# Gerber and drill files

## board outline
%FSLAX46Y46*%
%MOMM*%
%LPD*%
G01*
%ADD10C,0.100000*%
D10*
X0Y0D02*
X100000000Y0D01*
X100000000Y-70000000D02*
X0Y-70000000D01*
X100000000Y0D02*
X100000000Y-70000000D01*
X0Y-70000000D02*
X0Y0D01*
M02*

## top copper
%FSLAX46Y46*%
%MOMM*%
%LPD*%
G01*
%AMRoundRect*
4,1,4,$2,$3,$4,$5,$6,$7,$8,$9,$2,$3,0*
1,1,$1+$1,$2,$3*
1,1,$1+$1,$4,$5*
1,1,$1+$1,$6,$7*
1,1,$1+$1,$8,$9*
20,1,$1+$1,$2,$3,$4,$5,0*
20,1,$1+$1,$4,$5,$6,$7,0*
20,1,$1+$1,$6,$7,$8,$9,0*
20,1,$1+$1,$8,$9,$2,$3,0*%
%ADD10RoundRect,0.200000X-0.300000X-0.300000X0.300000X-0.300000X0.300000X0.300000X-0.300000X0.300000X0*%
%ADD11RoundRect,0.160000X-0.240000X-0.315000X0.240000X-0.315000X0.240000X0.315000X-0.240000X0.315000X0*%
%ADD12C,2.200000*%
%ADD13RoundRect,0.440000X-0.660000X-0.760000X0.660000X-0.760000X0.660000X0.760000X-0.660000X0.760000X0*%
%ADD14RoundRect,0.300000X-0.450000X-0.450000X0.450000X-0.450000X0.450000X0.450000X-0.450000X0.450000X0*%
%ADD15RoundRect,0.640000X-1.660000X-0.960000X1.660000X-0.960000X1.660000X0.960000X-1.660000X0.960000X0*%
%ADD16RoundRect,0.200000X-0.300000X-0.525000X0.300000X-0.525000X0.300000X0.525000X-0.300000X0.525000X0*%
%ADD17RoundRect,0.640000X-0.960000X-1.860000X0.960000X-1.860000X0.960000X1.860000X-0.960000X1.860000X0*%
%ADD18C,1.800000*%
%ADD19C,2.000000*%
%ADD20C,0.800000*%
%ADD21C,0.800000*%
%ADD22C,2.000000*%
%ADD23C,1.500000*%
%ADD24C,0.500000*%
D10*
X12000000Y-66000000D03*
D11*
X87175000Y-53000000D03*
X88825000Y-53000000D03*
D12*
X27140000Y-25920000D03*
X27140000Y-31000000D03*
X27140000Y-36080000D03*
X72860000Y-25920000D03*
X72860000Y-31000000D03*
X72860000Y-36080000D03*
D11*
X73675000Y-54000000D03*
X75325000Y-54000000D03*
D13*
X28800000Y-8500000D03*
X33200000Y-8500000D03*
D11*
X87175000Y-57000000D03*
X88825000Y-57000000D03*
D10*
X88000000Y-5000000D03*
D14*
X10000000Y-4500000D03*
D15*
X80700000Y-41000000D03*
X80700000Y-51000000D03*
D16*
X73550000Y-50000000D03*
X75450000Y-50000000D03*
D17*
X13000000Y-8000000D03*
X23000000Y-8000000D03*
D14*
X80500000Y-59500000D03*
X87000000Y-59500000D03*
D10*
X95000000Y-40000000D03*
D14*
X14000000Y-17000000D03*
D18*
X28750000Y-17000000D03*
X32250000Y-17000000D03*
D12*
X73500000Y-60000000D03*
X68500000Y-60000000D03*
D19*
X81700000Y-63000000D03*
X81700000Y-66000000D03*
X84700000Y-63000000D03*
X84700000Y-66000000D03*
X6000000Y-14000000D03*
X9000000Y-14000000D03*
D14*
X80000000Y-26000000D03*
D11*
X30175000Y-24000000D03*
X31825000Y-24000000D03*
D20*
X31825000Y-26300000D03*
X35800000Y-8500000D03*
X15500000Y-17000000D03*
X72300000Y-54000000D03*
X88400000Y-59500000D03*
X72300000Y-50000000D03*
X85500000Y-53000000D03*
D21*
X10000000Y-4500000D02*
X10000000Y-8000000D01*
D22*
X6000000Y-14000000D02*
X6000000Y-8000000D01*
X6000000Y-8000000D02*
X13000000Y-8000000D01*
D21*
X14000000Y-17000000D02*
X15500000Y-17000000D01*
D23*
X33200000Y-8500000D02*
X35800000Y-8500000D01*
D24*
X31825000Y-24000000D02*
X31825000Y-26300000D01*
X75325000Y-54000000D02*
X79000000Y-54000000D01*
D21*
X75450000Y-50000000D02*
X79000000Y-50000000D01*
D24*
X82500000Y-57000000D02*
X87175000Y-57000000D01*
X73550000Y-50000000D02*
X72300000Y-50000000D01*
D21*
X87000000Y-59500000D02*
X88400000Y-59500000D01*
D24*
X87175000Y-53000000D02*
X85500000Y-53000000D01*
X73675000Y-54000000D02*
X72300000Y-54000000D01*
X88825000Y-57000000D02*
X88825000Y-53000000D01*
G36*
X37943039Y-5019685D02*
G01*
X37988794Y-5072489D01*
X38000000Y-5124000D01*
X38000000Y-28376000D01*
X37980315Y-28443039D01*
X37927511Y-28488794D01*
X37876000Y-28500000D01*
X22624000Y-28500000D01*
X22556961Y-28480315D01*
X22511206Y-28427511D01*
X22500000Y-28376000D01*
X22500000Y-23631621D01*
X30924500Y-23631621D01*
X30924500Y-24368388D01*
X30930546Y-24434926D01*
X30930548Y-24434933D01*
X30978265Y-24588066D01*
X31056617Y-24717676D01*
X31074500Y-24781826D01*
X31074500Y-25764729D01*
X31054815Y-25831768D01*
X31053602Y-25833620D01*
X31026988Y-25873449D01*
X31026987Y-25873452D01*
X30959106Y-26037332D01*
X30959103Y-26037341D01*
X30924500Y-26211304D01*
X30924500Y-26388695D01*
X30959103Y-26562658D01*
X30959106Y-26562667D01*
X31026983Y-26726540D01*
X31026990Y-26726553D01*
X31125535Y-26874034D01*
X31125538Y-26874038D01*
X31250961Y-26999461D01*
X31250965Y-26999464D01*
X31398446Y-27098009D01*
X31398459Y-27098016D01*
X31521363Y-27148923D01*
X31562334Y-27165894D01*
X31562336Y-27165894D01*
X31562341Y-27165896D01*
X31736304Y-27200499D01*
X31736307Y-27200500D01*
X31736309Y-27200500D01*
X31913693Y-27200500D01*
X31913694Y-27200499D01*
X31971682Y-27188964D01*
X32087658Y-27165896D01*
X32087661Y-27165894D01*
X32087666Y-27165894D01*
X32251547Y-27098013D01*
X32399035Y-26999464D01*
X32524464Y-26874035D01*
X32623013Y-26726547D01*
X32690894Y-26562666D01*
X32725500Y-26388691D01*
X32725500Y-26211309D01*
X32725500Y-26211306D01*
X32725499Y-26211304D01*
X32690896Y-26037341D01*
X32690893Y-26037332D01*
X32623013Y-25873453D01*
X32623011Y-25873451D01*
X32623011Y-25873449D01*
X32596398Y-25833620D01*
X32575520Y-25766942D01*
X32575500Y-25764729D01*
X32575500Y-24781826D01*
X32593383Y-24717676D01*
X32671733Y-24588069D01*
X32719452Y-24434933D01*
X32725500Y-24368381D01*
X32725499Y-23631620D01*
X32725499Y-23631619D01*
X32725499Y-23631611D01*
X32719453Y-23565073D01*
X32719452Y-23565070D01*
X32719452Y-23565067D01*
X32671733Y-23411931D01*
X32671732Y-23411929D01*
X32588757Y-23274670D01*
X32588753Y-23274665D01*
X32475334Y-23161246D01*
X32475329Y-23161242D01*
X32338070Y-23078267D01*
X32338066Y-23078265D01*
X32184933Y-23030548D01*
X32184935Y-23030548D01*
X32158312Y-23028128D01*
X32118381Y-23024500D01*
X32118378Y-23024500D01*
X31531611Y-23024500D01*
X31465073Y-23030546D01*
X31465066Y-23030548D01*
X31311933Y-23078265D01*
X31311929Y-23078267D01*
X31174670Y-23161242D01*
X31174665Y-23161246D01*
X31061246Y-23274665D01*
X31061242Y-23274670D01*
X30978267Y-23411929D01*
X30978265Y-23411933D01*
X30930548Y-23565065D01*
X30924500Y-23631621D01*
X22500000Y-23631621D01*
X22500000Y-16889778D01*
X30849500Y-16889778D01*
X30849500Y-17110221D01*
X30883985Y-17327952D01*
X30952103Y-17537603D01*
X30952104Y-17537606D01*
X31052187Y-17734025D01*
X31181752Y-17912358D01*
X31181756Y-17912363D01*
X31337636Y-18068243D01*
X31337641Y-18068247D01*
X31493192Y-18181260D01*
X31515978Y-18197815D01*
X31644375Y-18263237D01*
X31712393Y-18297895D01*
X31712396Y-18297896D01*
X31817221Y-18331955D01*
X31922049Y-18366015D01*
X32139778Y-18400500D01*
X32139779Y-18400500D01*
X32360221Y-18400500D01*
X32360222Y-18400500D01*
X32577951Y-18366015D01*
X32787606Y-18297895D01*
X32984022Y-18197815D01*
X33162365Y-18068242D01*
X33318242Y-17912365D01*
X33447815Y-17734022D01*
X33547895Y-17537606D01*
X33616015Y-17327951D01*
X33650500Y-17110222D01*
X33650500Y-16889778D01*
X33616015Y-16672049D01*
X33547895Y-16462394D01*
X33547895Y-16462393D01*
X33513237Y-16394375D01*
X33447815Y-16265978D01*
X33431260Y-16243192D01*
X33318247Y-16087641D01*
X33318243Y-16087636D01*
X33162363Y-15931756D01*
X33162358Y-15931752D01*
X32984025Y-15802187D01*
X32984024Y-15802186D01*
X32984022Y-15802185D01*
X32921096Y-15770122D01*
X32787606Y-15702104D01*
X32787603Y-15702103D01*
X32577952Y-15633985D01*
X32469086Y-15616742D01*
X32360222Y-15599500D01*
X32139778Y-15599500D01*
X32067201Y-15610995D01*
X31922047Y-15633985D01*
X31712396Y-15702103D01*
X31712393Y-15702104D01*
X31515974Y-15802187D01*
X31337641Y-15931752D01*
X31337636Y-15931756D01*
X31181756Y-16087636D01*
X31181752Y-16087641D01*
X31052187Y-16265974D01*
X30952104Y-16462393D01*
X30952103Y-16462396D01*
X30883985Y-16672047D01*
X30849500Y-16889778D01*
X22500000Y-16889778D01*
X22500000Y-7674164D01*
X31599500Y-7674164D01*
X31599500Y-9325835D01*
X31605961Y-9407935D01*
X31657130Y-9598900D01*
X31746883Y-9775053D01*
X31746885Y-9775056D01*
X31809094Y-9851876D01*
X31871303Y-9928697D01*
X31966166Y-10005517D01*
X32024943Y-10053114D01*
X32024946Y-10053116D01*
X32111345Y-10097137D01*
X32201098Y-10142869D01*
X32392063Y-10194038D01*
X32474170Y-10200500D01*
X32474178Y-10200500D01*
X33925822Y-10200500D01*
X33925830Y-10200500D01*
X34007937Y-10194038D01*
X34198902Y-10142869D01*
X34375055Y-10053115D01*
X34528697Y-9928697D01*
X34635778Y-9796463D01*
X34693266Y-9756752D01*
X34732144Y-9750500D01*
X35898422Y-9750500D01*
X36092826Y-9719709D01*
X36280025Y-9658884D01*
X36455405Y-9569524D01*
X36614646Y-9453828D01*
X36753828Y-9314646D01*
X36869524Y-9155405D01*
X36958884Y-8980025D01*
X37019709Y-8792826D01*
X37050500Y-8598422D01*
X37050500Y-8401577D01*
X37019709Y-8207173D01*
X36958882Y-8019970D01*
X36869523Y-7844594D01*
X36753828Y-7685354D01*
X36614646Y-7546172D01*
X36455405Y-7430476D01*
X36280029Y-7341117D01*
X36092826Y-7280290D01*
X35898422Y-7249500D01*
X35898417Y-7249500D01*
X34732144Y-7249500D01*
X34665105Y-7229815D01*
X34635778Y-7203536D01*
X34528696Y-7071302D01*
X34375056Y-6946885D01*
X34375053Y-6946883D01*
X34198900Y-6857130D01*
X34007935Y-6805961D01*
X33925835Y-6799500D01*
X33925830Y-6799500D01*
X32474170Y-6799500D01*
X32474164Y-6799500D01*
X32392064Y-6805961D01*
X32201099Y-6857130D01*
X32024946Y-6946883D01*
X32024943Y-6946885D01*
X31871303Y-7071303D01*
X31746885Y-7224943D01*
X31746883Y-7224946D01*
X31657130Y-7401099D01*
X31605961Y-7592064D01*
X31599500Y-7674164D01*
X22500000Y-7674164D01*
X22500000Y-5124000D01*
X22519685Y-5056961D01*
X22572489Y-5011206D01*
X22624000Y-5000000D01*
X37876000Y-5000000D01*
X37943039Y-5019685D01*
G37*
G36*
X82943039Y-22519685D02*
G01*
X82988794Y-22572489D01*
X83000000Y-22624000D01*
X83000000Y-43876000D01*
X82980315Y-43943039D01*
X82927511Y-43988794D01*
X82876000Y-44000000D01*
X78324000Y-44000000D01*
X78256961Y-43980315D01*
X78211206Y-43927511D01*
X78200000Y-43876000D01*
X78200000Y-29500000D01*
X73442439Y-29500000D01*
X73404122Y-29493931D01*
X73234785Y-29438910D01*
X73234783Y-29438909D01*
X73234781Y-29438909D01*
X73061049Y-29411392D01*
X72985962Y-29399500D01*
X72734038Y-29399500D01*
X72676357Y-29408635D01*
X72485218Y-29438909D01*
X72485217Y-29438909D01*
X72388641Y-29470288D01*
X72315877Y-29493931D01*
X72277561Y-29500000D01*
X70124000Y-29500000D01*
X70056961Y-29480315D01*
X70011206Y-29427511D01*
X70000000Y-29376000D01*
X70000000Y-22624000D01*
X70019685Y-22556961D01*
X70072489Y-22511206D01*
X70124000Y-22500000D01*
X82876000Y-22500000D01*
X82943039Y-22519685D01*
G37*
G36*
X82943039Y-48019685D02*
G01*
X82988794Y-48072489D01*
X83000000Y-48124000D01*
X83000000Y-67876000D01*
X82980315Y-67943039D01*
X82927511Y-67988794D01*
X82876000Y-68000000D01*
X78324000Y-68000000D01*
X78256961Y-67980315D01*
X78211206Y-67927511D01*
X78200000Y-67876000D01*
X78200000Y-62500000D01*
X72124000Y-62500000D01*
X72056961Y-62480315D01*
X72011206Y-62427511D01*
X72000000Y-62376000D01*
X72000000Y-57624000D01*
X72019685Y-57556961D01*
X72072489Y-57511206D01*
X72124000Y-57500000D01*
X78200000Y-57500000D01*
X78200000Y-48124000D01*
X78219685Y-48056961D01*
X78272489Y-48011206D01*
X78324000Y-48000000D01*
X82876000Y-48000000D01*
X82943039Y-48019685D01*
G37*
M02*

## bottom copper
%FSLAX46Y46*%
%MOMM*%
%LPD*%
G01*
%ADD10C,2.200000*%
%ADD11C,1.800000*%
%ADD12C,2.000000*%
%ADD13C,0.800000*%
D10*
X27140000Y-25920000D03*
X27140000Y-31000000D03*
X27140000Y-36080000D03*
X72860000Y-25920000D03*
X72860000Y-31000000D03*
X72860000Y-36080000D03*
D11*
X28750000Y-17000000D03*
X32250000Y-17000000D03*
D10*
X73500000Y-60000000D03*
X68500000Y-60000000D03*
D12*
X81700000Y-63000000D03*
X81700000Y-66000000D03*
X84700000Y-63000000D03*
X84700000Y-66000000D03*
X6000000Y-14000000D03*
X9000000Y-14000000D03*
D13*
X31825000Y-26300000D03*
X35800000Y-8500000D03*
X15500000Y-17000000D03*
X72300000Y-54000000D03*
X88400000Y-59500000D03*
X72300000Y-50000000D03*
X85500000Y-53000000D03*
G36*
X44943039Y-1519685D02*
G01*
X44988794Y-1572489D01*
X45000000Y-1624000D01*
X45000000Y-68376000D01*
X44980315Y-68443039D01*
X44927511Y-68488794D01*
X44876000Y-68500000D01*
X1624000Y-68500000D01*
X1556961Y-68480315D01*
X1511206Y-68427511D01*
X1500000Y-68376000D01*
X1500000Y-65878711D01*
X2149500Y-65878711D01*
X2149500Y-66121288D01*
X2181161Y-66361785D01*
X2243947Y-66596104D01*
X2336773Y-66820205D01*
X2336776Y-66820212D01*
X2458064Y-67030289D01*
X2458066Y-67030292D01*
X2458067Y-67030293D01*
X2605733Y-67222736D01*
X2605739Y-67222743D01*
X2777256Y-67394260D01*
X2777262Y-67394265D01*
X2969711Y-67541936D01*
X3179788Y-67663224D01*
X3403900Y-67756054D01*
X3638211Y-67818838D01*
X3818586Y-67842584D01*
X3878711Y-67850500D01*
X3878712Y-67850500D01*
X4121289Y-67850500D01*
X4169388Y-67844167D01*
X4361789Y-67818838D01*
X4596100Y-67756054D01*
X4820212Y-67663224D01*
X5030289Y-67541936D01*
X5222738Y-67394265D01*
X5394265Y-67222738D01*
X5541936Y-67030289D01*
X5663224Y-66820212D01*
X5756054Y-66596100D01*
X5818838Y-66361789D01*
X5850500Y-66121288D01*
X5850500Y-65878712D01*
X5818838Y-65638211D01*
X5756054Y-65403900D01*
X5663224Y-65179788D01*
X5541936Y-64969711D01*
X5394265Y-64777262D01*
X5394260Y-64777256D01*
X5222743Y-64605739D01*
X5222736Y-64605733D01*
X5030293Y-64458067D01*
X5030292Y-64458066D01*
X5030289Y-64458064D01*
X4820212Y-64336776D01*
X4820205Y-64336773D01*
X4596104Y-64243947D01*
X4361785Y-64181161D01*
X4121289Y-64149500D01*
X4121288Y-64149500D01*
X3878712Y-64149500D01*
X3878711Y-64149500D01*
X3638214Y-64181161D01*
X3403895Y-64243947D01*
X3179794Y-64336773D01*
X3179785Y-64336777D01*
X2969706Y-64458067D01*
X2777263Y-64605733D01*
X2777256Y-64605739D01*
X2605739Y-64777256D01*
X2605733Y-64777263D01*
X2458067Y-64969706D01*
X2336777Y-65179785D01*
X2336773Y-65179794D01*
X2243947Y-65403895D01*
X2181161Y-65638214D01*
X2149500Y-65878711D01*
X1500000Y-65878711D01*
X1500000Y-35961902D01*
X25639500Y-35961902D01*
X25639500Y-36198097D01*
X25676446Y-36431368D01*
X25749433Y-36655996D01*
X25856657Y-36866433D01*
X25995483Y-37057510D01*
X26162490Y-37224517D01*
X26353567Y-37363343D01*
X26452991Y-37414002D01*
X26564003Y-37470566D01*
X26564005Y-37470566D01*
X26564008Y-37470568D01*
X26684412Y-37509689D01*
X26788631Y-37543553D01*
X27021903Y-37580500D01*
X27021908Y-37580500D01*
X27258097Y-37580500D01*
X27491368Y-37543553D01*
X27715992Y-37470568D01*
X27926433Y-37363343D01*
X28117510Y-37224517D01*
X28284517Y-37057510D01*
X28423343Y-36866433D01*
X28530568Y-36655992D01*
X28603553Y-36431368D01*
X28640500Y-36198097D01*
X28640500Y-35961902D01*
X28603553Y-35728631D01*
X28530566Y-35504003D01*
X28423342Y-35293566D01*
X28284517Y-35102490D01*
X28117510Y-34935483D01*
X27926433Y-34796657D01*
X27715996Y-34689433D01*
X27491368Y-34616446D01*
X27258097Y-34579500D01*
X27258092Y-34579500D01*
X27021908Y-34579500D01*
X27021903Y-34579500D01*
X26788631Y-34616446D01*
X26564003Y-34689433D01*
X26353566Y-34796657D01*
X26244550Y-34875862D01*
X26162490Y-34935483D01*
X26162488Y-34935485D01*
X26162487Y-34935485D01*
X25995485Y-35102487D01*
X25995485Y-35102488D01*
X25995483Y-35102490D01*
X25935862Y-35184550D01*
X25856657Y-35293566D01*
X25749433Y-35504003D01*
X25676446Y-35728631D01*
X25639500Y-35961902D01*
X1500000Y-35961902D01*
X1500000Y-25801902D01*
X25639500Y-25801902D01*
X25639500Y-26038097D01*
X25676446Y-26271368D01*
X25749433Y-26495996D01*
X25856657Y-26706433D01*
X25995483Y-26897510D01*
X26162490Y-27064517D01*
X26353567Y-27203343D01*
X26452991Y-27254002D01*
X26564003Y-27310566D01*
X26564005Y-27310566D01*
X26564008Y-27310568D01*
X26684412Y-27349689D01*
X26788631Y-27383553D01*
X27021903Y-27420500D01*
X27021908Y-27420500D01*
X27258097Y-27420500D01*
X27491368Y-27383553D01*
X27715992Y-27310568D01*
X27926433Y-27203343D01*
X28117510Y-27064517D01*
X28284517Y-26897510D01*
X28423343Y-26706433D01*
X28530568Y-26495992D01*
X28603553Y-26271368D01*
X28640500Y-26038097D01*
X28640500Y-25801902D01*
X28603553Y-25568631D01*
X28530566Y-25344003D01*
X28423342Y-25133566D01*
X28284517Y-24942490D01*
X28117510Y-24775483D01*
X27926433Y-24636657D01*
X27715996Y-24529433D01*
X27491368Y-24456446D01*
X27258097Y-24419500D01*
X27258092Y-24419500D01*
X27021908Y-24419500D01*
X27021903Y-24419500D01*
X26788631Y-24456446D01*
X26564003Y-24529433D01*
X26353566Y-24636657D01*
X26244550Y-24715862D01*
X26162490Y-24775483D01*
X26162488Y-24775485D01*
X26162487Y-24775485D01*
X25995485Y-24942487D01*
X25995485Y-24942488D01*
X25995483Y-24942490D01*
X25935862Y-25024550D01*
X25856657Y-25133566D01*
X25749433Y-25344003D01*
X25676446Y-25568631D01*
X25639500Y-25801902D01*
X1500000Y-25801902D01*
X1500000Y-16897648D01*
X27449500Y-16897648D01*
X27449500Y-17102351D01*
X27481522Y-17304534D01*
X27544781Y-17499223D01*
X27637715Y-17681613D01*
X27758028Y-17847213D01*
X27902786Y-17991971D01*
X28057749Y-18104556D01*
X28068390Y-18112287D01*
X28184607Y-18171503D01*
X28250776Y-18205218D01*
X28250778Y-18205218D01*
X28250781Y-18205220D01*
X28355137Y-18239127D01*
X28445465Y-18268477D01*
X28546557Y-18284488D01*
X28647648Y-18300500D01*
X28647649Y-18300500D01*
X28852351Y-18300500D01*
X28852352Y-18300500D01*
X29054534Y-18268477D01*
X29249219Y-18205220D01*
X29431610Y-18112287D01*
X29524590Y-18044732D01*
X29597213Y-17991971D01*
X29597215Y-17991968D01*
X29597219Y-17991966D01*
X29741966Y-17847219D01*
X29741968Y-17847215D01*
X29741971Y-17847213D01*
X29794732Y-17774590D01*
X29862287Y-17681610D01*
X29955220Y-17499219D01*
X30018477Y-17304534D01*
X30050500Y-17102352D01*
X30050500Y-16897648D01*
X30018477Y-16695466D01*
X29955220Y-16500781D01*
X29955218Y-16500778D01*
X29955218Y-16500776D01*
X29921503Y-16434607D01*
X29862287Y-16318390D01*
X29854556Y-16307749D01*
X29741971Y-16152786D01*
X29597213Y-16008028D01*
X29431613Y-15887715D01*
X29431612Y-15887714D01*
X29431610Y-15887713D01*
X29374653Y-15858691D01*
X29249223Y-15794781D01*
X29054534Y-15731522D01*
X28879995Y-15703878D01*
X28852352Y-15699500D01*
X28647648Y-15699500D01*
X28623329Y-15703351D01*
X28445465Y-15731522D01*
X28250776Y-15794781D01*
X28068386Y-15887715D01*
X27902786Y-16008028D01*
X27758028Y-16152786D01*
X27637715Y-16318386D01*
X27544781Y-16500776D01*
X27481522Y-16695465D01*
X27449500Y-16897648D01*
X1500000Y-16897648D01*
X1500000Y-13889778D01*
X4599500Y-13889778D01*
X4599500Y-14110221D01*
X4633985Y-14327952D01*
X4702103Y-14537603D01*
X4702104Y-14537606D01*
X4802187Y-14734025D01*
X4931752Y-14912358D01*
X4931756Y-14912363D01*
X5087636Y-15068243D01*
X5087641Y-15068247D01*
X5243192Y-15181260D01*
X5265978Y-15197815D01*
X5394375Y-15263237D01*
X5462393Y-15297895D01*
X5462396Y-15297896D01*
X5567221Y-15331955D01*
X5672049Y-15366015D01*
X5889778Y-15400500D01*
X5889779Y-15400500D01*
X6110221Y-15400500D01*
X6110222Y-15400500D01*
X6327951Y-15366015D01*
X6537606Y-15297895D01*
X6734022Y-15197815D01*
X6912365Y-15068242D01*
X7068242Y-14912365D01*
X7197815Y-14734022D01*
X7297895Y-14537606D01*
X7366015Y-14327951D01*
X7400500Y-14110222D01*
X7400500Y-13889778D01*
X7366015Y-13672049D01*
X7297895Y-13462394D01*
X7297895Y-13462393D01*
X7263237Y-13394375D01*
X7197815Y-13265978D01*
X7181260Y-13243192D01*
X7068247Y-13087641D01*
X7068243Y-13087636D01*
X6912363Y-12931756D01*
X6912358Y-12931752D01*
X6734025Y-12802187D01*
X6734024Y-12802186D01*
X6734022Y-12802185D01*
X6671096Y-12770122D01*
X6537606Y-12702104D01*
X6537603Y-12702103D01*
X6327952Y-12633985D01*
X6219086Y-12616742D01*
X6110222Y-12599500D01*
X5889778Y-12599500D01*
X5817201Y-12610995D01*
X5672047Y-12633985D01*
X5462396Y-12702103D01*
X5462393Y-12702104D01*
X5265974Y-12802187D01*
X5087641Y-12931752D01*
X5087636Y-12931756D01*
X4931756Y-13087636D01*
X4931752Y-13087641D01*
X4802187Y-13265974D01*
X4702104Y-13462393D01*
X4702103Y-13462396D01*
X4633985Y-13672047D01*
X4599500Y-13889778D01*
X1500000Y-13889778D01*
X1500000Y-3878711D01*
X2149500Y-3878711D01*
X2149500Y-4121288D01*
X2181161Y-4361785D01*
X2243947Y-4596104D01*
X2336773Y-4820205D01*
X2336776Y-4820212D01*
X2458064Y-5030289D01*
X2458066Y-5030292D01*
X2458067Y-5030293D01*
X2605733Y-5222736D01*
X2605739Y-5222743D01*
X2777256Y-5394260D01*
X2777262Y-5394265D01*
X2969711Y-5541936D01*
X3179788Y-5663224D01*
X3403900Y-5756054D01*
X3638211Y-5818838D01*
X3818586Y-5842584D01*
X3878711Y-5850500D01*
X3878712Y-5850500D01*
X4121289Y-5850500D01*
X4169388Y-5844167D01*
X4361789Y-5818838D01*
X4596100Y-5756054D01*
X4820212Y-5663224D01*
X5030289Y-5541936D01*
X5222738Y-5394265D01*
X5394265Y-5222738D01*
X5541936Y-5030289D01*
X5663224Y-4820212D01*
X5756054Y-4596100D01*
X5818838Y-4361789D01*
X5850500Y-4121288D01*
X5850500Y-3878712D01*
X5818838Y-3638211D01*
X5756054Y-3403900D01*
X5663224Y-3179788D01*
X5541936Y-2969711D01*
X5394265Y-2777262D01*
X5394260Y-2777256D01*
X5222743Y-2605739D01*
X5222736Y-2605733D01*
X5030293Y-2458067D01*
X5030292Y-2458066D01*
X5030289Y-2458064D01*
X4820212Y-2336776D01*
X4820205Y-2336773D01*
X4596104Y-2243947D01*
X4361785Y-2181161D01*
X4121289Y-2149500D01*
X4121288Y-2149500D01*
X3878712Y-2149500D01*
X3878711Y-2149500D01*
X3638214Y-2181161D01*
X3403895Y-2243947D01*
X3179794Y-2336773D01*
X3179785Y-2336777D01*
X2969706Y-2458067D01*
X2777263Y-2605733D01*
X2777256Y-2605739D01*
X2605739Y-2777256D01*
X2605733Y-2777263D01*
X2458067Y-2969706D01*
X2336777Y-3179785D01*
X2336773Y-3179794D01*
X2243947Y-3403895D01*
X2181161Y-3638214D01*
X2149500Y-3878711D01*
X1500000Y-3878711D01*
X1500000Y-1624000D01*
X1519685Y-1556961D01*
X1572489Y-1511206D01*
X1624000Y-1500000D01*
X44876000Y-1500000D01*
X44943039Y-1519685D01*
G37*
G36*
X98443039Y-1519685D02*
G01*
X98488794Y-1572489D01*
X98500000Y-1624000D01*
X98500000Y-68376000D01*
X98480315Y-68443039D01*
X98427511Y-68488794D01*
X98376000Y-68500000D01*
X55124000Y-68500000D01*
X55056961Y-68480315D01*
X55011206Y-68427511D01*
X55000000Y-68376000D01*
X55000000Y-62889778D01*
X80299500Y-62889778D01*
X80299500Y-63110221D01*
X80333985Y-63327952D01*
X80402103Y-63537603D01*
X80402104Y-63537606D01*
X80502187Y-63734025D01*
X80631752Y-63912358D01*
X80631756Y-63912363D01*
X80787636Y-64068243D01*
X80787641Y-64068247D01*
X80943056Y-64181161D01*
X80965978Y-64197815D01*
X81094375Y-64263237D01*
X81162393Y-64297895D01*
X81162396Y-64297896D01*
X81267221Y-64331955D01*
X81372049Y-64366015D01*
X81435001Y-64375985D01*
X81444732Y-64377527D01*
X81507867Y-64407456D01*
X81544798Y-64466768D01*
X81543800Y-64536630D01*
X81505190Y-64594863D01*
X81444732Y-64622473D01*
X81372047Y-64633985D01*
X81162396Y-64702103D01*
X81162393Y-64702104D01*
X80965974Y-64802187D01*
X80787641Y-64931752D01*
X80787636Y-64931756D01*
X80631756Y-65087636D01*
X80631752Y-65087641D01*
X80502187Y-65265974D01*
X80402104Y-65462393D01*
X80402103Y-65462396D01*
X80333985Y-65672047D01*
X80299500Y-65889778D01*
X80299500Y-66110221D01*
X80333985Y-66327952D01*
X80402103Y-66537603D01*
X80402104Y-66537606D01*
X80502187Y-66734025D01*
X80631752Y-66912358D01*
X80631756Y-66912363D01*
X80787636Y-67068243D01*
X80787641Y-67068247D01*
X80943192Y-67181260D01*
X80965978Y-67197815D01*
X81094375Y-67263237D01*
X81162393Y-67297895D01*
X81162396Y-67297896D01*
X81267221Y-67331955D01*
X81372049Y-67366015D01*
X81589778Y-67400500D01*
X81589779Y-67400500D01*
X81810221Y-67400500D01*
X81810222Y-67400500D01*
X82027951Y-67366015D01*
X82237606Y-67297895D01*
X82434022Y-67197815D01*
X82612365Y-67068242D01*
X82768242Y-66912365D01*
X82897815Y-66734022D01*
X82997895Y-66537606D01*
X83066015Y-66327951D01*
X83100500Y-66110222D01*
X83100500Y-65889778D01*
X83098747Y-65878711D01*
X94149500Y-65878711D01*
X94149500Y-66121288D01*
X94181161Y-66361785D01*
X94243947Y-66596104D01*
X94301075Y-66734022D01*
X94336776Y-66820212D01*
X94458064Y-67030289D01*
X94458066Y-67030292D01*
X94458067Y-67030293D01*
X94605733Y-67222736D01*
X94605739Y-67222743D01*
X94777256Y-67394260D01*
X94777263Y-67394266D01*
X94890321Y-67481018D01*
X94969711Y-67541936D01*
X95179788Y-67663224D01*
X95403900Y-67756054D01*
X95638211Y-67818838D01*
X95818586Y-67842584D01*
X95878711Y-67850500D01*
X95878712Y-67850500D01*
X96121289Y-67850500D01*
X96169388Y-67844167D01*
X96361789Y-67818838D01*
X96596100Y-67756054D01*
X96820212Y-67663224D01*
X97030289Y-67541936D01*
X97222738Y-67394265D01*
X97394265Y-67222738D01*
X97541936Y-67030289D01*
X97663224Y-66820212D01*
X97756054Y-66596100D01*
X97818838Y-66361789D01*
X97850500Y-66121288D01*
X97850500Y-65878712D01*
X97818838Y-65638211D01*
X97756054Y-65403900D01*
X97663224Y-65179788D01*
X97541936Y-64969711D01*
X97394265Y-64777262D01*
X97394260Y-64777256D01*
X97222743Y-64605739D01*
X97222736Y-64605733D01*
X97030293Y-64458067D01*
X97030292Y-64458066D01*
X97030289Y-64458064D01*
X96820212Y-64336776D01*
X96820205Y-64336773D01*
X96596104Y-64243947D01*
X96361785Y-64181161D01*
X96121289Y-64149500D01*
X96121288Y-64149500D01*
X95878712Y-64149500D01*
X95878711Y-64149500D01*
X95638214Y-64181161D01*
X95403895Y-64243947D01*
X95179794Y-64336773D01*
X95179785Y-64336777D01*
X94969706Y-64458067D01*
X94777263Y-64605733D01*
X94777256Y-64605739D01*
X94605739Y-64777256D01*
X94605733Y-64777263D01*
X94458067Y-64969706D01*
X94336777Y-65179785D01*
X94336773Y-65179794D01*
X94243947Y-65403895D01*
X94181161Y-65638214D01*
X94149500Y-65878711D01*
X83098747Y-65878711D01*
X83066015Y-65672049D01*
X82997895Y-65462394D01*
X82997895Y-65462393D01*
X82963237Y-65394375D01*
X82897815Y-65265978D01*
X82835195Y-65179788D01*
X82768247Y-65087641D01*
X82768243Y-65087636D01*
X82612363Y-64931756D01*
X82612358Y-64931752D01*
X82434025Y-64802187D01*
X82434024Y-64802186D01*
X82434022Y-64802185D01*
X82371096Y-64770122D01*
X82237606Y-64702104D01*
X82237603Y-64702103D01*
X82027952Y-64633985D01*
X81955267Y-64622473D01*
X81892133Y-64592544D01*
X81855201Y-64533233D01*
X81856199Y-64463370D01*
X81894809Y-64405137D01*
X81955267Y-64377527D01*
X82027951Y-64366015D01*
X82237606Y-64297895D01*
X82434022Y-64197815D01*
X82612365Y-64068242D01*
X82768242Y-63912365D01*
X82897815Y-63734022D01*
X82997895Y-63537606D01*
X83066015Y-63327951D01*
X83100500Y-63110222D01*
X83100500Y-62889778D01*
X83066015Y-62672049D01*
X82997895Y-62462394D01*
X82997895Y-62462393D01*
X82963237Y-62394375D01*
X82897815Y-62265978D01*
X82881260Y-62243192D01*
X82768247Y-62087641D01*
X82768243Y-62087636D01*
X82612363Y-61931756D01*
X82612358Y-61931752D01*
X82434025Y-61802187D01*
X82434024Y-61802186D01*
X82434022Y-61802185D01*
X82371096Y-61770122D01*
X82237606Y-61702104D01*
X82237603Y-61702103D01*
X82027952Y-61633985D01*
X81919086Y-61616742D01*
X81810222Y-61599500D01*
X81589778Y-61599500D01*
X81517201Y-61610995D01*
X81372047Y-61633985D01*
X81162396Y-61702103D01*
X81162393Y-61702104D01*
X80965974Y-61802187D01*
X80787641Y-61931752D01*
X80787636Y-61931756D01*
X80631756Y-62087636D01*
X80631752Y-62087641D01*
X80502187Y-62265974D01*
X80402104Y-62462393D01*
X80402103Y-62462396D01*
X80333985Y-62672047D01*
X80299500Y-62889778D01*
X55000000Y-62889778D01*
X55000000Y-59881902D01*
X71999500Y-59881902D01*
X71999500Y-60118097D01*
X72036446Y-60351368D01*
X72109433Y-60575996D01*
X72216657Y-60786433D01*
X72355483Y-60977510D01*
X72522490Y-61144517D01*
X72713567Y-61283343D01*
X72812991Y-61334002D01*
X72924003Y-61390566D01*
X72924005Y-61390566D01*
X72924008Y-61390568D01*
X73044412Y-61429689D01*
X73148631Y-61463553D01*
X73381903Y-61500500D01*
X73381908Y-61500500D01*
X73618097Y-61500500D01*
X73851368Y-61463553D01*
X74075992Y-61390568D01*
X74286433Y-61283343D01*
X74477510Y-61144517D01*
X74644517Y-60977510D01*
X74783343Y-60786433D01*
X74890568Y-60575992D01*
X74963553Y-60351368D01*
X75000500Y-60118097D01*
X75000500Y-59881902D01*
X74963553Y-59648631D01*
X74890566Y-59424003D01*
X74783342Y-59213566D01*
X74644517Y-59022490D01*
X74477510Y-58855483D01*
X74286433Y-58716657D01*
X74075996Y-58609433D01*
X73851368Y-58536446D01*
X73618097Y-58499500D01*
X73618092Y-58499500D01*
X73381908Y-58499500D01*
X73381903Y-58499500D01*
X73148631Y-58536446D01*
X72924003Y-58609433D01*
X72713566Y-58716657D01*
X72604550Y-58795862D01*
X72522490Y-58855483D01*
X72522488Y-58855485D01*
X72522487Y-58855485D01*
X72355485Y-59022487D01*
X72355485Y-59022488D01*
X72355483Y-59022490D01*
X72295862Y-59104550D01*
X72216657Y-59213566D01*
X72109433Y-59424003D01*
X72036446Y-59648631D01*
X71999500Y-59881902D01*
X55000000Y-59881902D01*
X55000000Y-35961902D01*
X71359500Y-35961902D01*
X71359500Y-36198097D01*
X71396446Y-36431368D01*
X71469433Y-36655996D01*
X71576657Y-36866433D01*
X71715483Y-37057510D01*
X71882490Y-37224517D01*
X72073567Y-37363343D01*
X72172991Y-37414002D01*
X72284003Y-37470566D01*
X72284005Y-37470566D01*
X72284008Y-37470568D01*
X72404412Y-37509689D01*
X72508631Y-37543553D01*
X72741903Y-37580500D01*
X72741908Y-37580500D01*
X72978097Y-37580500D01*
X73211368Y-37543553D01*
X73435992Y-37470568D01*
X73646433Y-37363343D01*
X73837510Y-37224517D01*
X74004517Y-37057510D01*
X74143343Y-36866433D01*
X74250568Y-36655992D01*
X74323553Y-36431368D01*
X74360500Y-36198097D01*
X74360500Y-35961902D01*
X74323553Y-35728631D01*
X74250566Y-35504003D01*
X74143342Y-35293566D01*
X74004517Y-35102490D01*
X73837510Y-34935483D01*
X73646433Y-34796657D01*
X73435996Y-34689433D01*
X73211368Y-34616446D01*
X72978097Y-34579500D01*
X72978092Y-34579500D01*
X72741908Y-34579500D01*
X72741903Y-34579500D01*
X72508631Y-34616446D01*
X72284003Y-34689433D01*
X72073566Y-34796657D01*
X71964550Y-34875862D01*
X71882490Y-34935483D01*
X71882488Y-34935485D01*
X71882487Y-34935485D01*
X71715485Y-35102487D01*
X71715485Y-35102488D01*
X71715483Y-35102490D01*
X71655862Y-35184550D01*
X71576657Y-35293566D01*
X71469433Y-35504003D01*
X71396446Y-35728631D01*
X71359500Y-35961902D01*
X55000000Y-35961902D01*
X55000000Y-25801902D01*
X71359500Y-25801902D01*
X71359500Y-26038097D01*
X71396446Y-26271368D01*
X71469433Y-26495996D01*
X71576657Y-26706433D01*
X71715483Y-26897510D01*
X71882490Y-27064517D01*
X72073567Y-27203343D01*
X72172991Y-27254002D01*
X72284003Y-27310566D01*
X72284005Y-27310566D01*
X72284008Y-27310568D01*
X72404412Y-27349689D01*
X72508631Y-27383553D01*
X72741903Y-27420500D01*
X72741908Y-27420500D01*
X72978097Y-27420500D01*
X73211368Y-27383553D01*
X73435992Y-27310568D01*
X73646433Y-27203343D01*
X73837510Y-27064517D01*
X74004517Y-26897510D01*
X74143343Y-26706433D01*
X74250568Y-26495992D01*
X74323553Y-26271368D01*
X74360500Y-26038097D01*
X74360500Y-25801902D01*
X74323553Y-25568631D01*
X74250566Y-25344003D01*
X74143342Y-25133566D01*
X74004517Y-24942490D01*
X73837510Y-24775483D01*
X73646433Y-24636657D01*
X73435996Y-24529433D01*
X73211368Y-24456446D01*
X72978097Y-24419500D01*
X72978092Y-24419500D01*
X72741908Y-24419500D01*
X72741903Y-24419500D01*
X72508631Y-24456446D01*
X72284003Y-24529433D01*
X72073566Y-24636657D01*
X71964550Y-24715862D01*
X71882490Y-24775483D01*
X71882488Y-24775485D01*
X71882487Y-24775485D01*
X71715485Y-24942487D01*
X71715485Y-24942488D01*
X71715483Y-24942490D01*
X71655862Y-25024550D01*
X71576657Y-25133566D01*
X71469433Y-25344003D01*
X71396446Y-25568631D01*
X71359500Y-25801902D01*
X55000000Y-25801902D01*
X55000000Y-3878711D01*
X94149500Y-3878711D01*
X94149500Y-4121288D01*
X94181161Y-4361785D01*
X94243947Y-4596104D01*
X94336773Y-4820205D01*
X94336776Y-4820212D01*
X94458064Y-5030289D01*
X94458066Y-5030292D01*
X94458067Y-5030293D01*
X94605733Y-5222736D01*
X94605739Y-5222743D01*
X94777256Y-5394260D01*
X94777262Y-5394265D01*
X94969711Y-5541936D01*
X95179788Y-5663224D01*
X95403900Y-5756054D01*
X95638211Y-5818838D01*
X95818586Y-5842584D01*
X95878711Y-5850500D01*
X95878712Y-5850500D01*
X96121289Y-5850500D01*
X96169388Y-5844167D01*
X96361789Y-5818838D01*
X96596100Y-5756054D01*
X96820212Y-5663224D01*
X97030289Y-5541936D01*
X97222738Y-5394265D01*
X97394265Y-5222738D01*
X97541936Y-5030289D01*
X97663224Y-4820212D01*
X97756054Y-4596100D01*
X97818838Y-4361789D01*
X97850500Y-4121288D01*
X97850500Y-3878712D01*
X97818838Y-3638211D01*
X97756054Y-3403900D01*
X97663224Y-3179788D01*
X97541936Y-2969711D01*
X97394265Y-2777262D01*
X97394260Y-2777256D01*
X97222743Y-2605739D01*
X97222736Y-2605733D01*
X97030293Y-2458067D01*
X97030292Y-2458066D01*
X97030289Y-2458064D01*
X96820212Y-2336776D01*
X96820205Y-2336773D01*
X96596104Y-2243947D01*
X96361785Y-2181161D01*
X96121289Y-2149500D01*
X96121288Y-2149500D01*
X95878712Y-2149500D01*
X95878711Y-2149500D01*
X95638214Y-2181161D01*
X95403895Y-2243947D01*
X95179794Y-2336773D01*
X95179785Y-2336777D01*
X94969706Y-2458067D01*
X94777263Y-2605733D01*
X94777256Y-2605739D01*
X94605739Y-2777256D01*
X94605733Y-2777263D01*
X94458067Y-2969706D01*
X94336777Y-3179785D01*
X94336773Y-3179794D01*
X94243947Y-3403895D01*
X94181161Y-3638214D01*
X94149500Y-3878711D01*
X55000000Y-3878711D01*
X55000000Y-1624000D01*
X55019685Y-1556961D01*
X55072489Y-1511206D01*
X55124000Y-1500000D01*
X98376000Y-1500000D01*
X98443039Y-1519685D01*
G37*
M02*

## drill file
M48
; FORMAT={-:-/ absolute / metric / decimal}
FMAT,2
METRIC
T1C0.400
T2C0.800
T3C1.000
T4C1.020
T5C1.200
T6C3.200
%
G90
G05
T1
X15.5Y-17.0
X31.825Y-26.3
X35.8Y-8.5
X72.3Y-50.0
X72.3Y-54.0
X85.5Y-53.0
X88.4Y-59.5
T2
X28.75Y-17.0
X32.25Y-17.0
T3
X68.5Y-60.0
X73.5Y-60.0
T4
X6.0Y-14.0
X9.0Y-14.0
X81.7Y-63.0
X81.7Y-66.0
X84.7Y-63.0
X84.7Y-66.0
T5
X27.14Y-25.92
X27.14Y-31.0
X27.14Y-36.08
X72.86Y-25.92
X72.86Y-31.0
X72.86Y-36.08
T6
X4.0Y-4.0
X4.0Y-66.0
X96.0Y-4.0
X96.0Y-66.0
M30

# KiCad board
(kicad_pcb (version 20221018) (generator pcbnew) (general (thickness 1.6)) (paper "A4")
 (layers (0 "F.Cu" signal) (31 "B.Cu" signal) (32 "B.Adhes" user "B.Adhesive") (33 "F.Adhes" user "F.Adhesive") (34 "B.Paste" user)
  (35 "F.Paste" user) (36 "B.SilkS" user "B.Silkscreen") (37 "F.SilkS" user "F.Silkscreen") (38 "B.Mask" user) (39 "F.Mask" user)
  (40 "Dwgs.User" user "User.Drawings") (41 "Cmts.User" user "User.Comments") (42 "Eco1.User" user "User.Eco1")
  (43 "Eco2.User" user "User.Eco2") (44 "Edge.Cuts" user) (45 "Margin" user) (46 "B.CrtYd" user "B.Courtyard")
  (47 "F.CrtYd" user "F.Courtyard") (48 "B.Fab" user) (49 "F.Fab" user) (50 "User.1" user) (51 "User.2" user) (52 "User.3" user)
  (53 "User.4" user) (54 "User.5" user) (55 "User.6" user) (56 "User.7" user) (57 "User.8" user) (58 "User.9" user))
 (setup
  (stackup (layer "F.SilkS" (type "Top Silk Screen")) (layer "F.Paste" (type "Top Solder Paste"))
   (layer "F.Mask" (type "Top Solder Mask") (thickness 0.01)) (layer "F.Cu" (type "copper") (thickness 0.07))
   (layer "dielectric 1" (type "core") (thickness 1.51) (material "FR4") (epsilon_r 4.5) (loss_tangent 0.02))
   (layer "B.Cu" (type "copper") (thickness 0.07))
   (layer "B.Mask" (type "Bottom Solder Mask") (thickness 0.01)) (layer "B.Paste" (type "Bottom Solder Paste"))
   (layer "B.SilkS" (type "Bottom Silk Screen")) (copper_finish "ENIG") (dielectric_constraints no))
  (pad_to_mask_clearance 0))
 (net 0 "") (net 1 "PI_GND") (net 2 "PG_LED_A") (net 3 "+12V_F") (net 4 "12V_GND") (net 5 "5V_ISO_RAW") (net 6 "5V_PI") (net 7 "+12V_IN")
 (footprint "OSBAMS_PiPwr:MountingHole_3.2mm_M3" (layer "F.Cu") (at 4 66)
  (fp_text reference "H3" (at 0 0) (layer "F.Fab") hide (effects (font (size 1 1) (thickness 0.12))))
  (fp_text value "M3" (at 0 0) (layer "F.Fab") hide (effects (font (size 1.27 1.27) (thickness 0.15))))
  (pad "" np_thru_hole circle (at 0 0) (size 3.2 3.2) (drill 3.2) (layers "F&B.Cu" "*.Mask")))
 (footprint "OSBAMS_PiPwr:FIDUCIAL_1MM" (layer "F.Cu") (at 12 66)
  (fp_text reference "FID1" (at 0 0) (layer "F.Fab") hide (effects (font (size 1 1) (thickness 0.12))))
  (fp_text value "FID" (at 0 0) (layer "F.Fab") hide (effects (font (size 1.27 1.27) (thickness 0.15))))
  (pad "1" smd roundrect (at 0 0) (size 1 1) (layers "F.Cu" "F.Mask") (roundrect_rratio 0.2) (solder_mask_margin 0.5)
   (thermal_bridge_angle 45)))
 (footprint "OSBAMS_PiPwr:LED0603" (layer "F.Cu") (at 88 53)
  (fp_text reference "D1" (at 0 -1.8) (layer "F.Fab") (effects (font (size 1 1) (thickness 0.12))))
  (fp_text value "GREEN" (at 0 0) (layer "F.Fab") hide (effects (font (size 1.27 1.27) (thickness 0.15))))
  (pad "1" smd roundrect (at -0.825 0) (size 0.8 0.95) (layers "F.Cu" "F.Paste" "F.Mask") (roundrect_rratio 0.2) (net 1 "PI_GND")
   (thermal_bridge_angle 45))
  (pad "2" smd roundrect (at 0.825 0) (size 0.8 0.95) (layers "F.Cu" "F.Paste" "F.Mask") (roundrect_rratio 0.2) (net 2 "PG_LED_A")
   (thermal_bridge_angle 45)))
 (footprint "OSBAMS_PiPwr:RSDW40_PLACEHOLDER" (layer "F.Cu") (at 50 31)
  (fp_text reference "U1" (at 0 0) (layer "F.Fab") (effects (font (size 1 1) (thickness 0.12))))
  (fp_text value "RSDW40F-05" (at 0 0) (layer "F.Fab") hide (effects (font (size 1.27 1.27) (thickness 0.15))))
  (pad "1" thru_hole circle (at -22.86 -5.08) (size 2.2 2.2) (drill 1.2) (layers "*.Cu" "*.Mask") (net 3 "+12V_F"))
  (pad "2" thru_hole circle (at -22.86 0) (size 2.2 2.2) (drill 1.2) (layers "*.Cu" "*.Mask") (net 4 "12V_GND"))
  (pad "3" thru_hole circle (at -22.86 5.08) (size 2.2 2.2) (drill 1.2) (layers "*.Cu" "*.Mask"))
  (pad "4" thru_hole circle (at 22.86 -5.08) (size 2.2 2.2) (drill 1.2) (layers "*.Cu" "*.Mask") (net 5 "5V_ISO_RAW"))
  (pad "5" thru_hole circle (at 22.86 0) (size 2.2 2.2) (drill 1.2) (layers "*.Cu" "*.Mask") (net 1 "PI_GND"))
  (pad "6" thru_hole circle (at 22.86 5.08) (size 2.2 2.2) (drill 1.2) (layers "*.Cu" "*.Mask")))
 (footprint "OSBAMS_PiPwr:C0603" (layer "F.Cu") (at 74.5 54)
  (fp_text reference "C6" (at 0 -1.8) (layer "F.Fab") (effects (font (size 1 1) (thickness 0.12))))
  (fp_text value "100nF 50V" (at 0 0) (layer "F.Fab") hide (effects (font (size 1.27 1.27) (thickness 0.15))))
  (pad "1" smd roundrect (at -0.825 0) (size 0.8 0.95) (layers "F.Cu" "F.Paste" "F.Mask") (roundrect_rratio 0.2) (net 1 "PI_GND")
   (thermal_bridge_angle 45))
  (pad "2" smd roundrect (at 0.825 0) (size 0.8 0.95) (layers "F.Cu" "F.Paste" "F.Mask") (roundrect_rratio 0.2) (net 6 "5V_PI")
   (thermal_bridge_angle 45)))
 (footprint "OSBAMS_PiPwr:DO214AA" (layer "F.Cu") (at 31 8.5)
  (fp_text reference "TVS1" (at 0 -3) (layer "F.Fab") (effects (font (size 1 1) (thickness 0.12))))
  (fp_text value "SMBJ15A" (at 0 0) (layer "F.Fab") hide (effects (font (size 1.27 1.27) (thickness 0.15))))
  (pad "1" smd roundrect (at -2.2 0) (size 2.2 2.4) (layers "F.Cu" "F.Paste" "F.Mask") (roundrect_rratio 0.2) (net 3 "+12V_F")
   (thermal_bridge_angle 45))
  (pad "2" smd roundrect (at 2.2 0) (size 2.2 2.4) (layers "F.Cu" "F.Paste" "F.Mask") (roundrect_rratio 0.2) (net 4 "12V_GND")
   (thermal_bridge_angle 45)))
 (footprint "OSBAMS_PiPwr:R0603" (layer "F.Cu") (at 88 57)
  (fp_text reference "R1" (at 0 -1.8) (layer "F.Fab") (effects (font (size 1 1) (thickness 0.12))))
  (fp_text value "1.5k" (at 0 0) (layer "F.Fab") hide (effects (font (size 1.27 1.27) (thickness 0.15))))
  (pad "1" smd roundrect (at -0.825 0) (size 0.8 0.95) (layers "F.Cu" "F.Paste" "F.Mask") (roundrect_rratio 0.2) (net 6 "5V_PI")
   (thermal_bridge_angle 45))
  (pad "2" smd roundrect (at 0.825 0) (size 0.8 0.95) (layers "F.Cu" "F.Paste" "F.Mask") (roundrect_rratio 0.2) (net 2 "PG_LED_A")
   (thermal_bridge_angle 45)))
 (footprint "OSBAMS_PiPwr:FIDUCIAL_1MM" (layer "F.Cu") (at 88 5)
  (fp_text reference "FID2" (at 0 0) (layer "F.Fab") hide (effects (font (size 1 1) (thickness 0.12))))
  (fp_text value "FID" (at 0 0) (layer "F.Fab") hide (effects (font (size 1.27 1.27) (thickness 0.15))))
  (pad "1" smd roundrect (at 0 0) (size 1 1) (layers "F.Cu" "F.Mask") (roundrect_rratio 0.2) (solder_mask_margin 0.5)
   (thermal_bridge_angle 45)))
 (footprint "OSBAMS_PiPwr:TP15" (layer "F.Cu") (at 10 4.5)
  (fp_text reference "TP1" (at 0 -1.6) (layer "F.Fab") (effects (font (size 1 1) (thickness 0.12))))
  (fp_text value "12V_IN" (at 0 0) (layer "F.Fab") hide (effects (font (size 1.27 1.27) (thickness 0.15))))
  (pad "1" smd roundrect (at 0 0) (size 1.5 1.5) (layers "F.Cu" "F.Paste" "F.Mask") (roundrect_rratio 0.2) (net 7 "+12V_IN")
   (thermal_bridge_angle 45)))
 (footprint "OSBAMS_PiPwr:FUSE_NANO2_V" (layer "F.Cu") (at 80.7 46)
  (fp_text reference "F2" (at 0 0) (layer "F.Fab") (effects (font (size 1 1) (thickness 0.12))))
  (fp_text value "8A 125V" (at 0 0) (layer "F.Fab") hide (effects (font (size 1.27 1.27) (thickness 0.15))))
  (pad "1" smd roundrect (at 0 -5) (size 4.6 3.2) (layers "F.Cu" "F.Paste" "F.Mask") (roundrect_rratio 0.2) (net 5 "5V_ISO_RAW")
   (thermal_bridge_angle 45))
  (pad "2" smd roundrect (at 0 5) (size 4.6 3.2) (layers "F.Cu" "F.Paste" "F.Mask") (roundrect_rratio 0.2) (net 6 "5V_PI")
   (thermal_bridge_angle 45)))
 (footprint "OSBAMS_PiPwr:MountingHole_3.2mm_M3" (layer "F.Cu") (at 96 66)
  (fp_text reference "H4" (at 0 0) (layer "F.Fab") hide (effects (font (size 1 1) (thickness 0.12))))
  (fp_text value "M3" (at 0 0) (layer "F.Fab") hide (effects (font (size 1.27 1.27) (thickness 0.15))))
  (pad "" np_thru_hole circle (at 0 0) (size 3.2 3.2) (drill 3.2) (layers "F&B.Cu" "*.Mask")))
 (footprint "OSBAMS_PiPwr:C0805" (layer "F.Cu") (at 74.5 50)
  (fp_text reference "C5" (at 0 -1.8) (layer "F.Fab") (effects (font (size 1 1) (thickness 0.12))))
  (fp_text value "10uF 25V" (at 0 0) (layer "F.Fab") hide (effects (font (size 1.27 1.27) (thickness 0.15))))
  (pad "1" smd roundrect (at -0.95 0) (size 1 1.45) (layers "F.Cu" "F.Paste" "F.Mask") (roundrect_rratio 0.2) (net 1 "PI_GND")
   (thermal_bridge_angle 45))
  (pad "2" smd roundrect (at 0.95 0) (size 1 1.45) (layers "F.Cu" "F.Paste" "F.Mask") (roundrect_rratio 0.2) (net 6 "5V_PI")
   (thermal_bridge_angle 45)))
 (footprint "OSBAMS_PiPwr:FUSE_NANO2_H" (layer "F.Cu") (at 18 8)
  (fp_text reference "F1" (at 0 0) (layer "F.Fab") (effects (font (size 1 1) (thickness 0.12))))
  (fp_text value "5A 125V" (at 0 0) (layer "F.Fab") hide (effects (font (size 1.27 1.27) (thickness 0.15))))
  (pad "1" smd roundrect (at -5 0) (size 3.2 5) (layers "F.Cu" "F.Paste" "F.Mask") (roundrect_rratio 0.2) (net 7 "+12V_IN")
   (thermal_bridge_angle 45))
  (pad "2" smd roundrect (at 5 0) (size 3.2 5) (layers "F.Cu" "F.Paste" "F.Mask") (roundrect_rratio 0.2) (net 3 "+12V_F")
   (thermal_bridge_angle 45)))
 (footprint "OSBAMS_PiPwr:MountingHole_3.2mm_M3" (layer "F.Cu") (at 4 4)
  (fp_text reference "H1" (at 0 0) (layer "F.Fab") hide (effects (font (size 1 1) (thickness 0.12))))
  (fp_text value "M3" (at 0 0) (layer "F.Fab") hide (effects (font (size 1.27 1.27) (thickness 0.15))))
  (pad "" np_thru_hole circle (at 0 0) (size 3.2 3.2) (drill 3.2) (layers "F&B.Cu" "*.Mask")))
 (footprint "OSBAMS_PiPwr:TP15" (layer "F.Cu") (at 80.5 59.5)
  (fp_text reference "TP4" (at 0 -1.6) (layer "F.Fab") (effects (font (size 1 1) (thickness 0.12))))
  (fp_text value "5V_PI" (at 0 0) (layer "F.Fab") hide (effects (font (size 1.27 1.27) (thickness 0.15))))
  (pad "1" smd roundrect (at 0 0) (size 1.5 1.5) (layers "F.Cu" "F.Paste" "F.Mask") (roundrect_rratio 0.2) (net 6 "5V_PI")
   (thermal_bridge_angle 45)))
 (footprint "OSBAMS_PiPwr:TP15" (layer "F.Cu") (at 87 59.5)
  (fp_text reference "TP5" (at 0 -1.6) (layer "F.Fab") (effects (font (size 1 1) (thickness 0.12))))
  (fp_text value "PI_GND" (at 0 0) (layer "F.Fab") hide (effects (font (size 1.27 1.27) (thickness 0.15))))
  (pad "1" smd roundrect (at 0 0) (size 1.5 1.5) (layers "F.Cu" "F.Paste" "F.Mask") (roundrect_rratio 0.2) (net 1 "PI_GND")
   (thermal_bridge_angle 45)))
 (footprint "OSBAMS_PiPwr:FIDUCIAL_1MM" (layer "F.Cu") (at 95 40)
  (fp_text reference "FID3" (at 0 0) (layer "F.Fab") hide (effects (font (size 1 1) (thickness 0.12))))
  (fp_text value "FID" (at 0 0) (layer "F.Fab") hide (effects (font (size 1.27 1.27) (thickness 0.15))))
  (pad "1" smd roundrect (at 0 0) (size 1 1) (layers "F.Cu" "F.Mask") (roundrect_rratio 0.2) (solder_mask_margin 0.5)
   (thermal_bridge_angle 45)))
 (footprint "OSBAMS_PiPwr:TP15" (layer "F.Cu") (at 14 17)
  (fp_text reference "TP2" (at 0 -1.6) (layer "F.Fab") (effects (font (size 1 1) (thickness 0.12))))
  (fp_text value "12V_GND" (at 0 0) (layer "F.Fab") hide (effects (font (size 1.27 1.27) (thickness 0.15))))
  (pad "1" smd roundrect (at 0 0) (size 1.5 1.5) (layers "F.Cu" "F.Paste" "F.Mask") (roundrect_rratio 0.2) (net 4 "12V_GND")
   (thermal_bridge_angle 45)))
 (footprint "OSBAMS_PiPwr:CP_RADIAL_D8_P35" (layer "F.Cu") (at 30.5 17)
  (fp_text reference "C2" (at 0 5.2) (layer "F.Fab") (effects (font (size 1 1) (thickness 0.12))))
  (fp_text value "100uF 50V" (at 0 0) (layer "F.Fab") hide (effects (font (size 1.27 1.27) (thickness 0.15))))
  (pad "1" thru_hole circle (at -1.75 0) (size 1.8 1.8) (drill 0.8) (layers "*.Cu" "*.Mask") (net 3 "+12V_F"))
  (pad "2" thru_hole circle (at 1.75 0) (size 1.8 1.8) (drill 0.8) (layers "*.Cu" "*.Mask") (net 4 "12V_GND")))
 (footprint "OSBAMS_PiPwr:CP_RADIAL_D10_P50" (layer "F.Cu") (at 71 60)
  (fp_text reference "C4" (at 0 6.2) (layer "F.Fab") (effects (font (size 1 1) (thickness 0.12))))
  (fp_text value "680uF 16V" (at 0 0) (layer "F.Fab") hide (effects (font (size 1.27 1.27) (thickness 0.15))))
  (pad "1" thru_hole circle (at 2.5 0) (size 2.2 2.2) (drill 1) (layers "*.Cu" "*.Mask") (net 6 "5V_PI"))
  (pad "2" thru_hole circle (at -2.5 0) (size 2.2 2.2) (drill 1) (layers "*.Cu" "*.Mask") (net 1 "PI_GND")))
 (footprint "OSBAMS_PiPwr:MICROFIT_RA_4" (layer "F.Cu") (at 81.7 63)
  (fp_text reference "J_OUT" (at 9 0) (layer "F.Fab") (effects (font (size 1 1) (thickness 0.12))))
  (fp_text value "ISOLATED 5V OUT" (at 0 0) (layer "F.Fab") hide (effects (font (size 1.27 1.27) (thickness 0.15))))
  (pad "1" thru_hole circle (at 0 0) (size 2 2) (drill 1.02) (layers "*.Cu" "*.Mask") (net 6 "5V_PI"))
  (pad "2" thru_hole circle (at 0 3) (size 2 2) (drill 1.02) (layers "*.Cu" "*.Mask") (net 6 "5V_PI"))
  (pad "3" thru_hole circle (at 3 0) (size 2 2) (drill 1.02) (layers "*.Cu" "*.Mask") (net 1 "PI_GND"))
  (pad "4" thru_hole circle (at 3 3) (size 2 2) (drill 1.02) (layers "*.Cu" "*.Mask") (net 1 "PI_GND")))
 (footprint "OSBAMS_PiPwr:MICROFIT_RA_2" (layer "F.Cu") (at 6 14)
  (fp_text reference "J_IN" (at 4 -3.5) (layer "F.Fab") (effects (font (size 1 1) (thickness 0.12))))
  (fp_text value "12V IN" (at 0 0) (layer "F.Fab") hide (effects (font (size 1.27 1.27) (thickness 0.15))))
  (pad "1" thru_hole circle (at 0 0) (size 2 2) (drill 1.02) (layers "*.Cu" "*.Mask") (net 7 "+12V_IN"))
  (pad "2" thru_hole circle (at 3 0) (size 2 2) (drill 1.02) (layers "*.Cu" "*.Mask") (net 4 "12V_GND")))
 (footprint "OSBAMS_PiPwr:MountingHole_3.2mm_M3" (layer "F.Cu") (at 96 4)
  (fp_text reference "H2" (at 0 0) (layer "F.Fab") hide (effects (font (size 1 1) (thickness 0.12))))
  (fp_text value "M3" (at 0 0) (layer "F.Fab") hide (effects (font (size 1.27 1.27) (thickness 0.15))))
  (pad "" np_thru_hole circle (at 0 0) (size 3.2 3.2) (drill 3.2) (layers "F&B.Cu" "*.Mask")))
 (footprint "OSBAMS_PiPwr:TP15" (layer "F.Cu") (at 80 26)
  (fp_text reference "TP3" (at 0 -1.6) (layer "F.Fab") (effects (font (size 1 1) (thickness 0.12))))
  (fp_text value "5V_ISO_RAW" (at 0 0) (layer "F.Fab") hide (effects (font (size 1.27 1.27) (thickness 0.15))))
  (pad "1" smd roundrect (at 0 0) (size 1.5 1.5) (layers "F.Cu" "F.Paste" "F.Mask") (roundrect_rratio 0.2) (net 5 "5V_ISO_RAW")
   (thermal_bridge_angle 45)))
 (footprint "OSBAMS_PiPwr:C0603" (layer "F.Cu") (at 31 24)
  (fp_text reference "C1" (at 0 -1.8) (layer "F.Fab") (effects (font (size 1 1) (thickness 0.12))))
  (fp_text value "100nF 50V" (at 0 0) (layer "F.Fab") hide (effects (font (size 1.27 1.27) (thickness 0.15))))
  (pad "1" smd roundrect (at -0.825 0) (size 0.8 0.95) (layers "F.Cu" "F.Paste" "F.Mask") (roundrect_rratio 0.2) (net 3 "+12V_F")
   (thermal_bridge_angle 45))
  (pad "2" smd roundrect (at 0.825 0) (size 0.8 0.95) (layers "F.Cu" "F.Paste" "F.Mask") (roundrect_rratio 0.2) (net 4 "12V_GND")
   (thermal_bridge_angle 45)))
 (gr_line (start 0 0) (end 100 0) (stroke (width 0.1) (type default)) (layer "Edge.Cuts"))
 (gr_line (start 100 70) (end 0 70) (stroke (width 0.1) (type default)) (layer "Edge.Cuts"))
 (gr_line (start 100 0) (end 100 70) (stroke (width 0.1) (type default)) (layer "Edge.Cuts"))
 (gr_line (start 0 70) (end 0 0) (stroke (width 0.1) (type default)) (layer "Edge.Cuts"))
 (segment (start 10 4.5) (end 10 8) (width 0.8) (layer "F.Cu") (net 7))
 (segment (start 6 14) (end 6 8) (width 2) (layer "F.Cu") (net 7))
 (segment (start 6 8) (end 13 8) (width 2) (layer "F.Cu") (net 7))
 (segment (start 14 17) (end 15.5 17) (width 0.8) (layer "F.Cu") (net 4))
 (segment (start 33.2 8.5) (end 35.8 8.5) (width 1.5) (layer "F.Cu") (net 4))
 (segment (start 31.825 24) (end 31.825 26.3) (width 0.5) (layer "F.Cu") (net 4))
 (via (at 31.825 26.3) (size 0.8) (drill 0.4) (layers "F.Cu" "B.Cu") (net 4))
 (via (at 35.8 8.5) (size 0.8) (drill 0.4) (layers "F.Cu" "B.Cu") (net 4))
 (via (at 15.5 17) (size 0.8) (drill 0.4) (layers "F.Cu" "B.Cu") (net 4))
 (segment (start 75.325 54) (end 79 54) (width 0.5) (layer "F.Cu") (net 6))
 (segment (start 75.45 50) (end 79 50) (width 0.8) (layer "F.Cu") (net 6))
 (segment (start 82.5 57) (end 87.175 57) (width 0.5) (layer "F.Cu") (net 6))
 (segment (start 73.55 50) (end 72.3 50) (width 0.5) (layer "F.Cu") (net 1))
 (segment (start 87 59.5) (end 88.4 59.5) (width 0.8) (layer "F.Cu") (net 1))
 (segment (start 87.175 53) (end 85.5 53) (width 0.5) (layer "F.Cu") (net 1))
 (segment (start 73.675 54) (end 72.3 54) (width 0.5) (layer "F.Cu") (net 1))
 (via (at 72.3 54) (size 0.8) (drill 0.4) (layers "F.Cu" "B.Cu") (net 1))
 (via (at 88.4 59.5) (size 0.8) (drill 0.4) (layers "F.Cu" "B.Cu") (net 1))
 (via (at 72.3 50) (size 0.8) (drill 0.4) (layers "F.Cu" "B.Cu") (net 1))
 (via (at 85.5 53) (size 0.8) (drill 0.4) (layers "F.Cu" "B.Cu") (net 1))
 (segment (start 88.825 57) (end 88.825 53) (width 0.5) (layer "F.Cu") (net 2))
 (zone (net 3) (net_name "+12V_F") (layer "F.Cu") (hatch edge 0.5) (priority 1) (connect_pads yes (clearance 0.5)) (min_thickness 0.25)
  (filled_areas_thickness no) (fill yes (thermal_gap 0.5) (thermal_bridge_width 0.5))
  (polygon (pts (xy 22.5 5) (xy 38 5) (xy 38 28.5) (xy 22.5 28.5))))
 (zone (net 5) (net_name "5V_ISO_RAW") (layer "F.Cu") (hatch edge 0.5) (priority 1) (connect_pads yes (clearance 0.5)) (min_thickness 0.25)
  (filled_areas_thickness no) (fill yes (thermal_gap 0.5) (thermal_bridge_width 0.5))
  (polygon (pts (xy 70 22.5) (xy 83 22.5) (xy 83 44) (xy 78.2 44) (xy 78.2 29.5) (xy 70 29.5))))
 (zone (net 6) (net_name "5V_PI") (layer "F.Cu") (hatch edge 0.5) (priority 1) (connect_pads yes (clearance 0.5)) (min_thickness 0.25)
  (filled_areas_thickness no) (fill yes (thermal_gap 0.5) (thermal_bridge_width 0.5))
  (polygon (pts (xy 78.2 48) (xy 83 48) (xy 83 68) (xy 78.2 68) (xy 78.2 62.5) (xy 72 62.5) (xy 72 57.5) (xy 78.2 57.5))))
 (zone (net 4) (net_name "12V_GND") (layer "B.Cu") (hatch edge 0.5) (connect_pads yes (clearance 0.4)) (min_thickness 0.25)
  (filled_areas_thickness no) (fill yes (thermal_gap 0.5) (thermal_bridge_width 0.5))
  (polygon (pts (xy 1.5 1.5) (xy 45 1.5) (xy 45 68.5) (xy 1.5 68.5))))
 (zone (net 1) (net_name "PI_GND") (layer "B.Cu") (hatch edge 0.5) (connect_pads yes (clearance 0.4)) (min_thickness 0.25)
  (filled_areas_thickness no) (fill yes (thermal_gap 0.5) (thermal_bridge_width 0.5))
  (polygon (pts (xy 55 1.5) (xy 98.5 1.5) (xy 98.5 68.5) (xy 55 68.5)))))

